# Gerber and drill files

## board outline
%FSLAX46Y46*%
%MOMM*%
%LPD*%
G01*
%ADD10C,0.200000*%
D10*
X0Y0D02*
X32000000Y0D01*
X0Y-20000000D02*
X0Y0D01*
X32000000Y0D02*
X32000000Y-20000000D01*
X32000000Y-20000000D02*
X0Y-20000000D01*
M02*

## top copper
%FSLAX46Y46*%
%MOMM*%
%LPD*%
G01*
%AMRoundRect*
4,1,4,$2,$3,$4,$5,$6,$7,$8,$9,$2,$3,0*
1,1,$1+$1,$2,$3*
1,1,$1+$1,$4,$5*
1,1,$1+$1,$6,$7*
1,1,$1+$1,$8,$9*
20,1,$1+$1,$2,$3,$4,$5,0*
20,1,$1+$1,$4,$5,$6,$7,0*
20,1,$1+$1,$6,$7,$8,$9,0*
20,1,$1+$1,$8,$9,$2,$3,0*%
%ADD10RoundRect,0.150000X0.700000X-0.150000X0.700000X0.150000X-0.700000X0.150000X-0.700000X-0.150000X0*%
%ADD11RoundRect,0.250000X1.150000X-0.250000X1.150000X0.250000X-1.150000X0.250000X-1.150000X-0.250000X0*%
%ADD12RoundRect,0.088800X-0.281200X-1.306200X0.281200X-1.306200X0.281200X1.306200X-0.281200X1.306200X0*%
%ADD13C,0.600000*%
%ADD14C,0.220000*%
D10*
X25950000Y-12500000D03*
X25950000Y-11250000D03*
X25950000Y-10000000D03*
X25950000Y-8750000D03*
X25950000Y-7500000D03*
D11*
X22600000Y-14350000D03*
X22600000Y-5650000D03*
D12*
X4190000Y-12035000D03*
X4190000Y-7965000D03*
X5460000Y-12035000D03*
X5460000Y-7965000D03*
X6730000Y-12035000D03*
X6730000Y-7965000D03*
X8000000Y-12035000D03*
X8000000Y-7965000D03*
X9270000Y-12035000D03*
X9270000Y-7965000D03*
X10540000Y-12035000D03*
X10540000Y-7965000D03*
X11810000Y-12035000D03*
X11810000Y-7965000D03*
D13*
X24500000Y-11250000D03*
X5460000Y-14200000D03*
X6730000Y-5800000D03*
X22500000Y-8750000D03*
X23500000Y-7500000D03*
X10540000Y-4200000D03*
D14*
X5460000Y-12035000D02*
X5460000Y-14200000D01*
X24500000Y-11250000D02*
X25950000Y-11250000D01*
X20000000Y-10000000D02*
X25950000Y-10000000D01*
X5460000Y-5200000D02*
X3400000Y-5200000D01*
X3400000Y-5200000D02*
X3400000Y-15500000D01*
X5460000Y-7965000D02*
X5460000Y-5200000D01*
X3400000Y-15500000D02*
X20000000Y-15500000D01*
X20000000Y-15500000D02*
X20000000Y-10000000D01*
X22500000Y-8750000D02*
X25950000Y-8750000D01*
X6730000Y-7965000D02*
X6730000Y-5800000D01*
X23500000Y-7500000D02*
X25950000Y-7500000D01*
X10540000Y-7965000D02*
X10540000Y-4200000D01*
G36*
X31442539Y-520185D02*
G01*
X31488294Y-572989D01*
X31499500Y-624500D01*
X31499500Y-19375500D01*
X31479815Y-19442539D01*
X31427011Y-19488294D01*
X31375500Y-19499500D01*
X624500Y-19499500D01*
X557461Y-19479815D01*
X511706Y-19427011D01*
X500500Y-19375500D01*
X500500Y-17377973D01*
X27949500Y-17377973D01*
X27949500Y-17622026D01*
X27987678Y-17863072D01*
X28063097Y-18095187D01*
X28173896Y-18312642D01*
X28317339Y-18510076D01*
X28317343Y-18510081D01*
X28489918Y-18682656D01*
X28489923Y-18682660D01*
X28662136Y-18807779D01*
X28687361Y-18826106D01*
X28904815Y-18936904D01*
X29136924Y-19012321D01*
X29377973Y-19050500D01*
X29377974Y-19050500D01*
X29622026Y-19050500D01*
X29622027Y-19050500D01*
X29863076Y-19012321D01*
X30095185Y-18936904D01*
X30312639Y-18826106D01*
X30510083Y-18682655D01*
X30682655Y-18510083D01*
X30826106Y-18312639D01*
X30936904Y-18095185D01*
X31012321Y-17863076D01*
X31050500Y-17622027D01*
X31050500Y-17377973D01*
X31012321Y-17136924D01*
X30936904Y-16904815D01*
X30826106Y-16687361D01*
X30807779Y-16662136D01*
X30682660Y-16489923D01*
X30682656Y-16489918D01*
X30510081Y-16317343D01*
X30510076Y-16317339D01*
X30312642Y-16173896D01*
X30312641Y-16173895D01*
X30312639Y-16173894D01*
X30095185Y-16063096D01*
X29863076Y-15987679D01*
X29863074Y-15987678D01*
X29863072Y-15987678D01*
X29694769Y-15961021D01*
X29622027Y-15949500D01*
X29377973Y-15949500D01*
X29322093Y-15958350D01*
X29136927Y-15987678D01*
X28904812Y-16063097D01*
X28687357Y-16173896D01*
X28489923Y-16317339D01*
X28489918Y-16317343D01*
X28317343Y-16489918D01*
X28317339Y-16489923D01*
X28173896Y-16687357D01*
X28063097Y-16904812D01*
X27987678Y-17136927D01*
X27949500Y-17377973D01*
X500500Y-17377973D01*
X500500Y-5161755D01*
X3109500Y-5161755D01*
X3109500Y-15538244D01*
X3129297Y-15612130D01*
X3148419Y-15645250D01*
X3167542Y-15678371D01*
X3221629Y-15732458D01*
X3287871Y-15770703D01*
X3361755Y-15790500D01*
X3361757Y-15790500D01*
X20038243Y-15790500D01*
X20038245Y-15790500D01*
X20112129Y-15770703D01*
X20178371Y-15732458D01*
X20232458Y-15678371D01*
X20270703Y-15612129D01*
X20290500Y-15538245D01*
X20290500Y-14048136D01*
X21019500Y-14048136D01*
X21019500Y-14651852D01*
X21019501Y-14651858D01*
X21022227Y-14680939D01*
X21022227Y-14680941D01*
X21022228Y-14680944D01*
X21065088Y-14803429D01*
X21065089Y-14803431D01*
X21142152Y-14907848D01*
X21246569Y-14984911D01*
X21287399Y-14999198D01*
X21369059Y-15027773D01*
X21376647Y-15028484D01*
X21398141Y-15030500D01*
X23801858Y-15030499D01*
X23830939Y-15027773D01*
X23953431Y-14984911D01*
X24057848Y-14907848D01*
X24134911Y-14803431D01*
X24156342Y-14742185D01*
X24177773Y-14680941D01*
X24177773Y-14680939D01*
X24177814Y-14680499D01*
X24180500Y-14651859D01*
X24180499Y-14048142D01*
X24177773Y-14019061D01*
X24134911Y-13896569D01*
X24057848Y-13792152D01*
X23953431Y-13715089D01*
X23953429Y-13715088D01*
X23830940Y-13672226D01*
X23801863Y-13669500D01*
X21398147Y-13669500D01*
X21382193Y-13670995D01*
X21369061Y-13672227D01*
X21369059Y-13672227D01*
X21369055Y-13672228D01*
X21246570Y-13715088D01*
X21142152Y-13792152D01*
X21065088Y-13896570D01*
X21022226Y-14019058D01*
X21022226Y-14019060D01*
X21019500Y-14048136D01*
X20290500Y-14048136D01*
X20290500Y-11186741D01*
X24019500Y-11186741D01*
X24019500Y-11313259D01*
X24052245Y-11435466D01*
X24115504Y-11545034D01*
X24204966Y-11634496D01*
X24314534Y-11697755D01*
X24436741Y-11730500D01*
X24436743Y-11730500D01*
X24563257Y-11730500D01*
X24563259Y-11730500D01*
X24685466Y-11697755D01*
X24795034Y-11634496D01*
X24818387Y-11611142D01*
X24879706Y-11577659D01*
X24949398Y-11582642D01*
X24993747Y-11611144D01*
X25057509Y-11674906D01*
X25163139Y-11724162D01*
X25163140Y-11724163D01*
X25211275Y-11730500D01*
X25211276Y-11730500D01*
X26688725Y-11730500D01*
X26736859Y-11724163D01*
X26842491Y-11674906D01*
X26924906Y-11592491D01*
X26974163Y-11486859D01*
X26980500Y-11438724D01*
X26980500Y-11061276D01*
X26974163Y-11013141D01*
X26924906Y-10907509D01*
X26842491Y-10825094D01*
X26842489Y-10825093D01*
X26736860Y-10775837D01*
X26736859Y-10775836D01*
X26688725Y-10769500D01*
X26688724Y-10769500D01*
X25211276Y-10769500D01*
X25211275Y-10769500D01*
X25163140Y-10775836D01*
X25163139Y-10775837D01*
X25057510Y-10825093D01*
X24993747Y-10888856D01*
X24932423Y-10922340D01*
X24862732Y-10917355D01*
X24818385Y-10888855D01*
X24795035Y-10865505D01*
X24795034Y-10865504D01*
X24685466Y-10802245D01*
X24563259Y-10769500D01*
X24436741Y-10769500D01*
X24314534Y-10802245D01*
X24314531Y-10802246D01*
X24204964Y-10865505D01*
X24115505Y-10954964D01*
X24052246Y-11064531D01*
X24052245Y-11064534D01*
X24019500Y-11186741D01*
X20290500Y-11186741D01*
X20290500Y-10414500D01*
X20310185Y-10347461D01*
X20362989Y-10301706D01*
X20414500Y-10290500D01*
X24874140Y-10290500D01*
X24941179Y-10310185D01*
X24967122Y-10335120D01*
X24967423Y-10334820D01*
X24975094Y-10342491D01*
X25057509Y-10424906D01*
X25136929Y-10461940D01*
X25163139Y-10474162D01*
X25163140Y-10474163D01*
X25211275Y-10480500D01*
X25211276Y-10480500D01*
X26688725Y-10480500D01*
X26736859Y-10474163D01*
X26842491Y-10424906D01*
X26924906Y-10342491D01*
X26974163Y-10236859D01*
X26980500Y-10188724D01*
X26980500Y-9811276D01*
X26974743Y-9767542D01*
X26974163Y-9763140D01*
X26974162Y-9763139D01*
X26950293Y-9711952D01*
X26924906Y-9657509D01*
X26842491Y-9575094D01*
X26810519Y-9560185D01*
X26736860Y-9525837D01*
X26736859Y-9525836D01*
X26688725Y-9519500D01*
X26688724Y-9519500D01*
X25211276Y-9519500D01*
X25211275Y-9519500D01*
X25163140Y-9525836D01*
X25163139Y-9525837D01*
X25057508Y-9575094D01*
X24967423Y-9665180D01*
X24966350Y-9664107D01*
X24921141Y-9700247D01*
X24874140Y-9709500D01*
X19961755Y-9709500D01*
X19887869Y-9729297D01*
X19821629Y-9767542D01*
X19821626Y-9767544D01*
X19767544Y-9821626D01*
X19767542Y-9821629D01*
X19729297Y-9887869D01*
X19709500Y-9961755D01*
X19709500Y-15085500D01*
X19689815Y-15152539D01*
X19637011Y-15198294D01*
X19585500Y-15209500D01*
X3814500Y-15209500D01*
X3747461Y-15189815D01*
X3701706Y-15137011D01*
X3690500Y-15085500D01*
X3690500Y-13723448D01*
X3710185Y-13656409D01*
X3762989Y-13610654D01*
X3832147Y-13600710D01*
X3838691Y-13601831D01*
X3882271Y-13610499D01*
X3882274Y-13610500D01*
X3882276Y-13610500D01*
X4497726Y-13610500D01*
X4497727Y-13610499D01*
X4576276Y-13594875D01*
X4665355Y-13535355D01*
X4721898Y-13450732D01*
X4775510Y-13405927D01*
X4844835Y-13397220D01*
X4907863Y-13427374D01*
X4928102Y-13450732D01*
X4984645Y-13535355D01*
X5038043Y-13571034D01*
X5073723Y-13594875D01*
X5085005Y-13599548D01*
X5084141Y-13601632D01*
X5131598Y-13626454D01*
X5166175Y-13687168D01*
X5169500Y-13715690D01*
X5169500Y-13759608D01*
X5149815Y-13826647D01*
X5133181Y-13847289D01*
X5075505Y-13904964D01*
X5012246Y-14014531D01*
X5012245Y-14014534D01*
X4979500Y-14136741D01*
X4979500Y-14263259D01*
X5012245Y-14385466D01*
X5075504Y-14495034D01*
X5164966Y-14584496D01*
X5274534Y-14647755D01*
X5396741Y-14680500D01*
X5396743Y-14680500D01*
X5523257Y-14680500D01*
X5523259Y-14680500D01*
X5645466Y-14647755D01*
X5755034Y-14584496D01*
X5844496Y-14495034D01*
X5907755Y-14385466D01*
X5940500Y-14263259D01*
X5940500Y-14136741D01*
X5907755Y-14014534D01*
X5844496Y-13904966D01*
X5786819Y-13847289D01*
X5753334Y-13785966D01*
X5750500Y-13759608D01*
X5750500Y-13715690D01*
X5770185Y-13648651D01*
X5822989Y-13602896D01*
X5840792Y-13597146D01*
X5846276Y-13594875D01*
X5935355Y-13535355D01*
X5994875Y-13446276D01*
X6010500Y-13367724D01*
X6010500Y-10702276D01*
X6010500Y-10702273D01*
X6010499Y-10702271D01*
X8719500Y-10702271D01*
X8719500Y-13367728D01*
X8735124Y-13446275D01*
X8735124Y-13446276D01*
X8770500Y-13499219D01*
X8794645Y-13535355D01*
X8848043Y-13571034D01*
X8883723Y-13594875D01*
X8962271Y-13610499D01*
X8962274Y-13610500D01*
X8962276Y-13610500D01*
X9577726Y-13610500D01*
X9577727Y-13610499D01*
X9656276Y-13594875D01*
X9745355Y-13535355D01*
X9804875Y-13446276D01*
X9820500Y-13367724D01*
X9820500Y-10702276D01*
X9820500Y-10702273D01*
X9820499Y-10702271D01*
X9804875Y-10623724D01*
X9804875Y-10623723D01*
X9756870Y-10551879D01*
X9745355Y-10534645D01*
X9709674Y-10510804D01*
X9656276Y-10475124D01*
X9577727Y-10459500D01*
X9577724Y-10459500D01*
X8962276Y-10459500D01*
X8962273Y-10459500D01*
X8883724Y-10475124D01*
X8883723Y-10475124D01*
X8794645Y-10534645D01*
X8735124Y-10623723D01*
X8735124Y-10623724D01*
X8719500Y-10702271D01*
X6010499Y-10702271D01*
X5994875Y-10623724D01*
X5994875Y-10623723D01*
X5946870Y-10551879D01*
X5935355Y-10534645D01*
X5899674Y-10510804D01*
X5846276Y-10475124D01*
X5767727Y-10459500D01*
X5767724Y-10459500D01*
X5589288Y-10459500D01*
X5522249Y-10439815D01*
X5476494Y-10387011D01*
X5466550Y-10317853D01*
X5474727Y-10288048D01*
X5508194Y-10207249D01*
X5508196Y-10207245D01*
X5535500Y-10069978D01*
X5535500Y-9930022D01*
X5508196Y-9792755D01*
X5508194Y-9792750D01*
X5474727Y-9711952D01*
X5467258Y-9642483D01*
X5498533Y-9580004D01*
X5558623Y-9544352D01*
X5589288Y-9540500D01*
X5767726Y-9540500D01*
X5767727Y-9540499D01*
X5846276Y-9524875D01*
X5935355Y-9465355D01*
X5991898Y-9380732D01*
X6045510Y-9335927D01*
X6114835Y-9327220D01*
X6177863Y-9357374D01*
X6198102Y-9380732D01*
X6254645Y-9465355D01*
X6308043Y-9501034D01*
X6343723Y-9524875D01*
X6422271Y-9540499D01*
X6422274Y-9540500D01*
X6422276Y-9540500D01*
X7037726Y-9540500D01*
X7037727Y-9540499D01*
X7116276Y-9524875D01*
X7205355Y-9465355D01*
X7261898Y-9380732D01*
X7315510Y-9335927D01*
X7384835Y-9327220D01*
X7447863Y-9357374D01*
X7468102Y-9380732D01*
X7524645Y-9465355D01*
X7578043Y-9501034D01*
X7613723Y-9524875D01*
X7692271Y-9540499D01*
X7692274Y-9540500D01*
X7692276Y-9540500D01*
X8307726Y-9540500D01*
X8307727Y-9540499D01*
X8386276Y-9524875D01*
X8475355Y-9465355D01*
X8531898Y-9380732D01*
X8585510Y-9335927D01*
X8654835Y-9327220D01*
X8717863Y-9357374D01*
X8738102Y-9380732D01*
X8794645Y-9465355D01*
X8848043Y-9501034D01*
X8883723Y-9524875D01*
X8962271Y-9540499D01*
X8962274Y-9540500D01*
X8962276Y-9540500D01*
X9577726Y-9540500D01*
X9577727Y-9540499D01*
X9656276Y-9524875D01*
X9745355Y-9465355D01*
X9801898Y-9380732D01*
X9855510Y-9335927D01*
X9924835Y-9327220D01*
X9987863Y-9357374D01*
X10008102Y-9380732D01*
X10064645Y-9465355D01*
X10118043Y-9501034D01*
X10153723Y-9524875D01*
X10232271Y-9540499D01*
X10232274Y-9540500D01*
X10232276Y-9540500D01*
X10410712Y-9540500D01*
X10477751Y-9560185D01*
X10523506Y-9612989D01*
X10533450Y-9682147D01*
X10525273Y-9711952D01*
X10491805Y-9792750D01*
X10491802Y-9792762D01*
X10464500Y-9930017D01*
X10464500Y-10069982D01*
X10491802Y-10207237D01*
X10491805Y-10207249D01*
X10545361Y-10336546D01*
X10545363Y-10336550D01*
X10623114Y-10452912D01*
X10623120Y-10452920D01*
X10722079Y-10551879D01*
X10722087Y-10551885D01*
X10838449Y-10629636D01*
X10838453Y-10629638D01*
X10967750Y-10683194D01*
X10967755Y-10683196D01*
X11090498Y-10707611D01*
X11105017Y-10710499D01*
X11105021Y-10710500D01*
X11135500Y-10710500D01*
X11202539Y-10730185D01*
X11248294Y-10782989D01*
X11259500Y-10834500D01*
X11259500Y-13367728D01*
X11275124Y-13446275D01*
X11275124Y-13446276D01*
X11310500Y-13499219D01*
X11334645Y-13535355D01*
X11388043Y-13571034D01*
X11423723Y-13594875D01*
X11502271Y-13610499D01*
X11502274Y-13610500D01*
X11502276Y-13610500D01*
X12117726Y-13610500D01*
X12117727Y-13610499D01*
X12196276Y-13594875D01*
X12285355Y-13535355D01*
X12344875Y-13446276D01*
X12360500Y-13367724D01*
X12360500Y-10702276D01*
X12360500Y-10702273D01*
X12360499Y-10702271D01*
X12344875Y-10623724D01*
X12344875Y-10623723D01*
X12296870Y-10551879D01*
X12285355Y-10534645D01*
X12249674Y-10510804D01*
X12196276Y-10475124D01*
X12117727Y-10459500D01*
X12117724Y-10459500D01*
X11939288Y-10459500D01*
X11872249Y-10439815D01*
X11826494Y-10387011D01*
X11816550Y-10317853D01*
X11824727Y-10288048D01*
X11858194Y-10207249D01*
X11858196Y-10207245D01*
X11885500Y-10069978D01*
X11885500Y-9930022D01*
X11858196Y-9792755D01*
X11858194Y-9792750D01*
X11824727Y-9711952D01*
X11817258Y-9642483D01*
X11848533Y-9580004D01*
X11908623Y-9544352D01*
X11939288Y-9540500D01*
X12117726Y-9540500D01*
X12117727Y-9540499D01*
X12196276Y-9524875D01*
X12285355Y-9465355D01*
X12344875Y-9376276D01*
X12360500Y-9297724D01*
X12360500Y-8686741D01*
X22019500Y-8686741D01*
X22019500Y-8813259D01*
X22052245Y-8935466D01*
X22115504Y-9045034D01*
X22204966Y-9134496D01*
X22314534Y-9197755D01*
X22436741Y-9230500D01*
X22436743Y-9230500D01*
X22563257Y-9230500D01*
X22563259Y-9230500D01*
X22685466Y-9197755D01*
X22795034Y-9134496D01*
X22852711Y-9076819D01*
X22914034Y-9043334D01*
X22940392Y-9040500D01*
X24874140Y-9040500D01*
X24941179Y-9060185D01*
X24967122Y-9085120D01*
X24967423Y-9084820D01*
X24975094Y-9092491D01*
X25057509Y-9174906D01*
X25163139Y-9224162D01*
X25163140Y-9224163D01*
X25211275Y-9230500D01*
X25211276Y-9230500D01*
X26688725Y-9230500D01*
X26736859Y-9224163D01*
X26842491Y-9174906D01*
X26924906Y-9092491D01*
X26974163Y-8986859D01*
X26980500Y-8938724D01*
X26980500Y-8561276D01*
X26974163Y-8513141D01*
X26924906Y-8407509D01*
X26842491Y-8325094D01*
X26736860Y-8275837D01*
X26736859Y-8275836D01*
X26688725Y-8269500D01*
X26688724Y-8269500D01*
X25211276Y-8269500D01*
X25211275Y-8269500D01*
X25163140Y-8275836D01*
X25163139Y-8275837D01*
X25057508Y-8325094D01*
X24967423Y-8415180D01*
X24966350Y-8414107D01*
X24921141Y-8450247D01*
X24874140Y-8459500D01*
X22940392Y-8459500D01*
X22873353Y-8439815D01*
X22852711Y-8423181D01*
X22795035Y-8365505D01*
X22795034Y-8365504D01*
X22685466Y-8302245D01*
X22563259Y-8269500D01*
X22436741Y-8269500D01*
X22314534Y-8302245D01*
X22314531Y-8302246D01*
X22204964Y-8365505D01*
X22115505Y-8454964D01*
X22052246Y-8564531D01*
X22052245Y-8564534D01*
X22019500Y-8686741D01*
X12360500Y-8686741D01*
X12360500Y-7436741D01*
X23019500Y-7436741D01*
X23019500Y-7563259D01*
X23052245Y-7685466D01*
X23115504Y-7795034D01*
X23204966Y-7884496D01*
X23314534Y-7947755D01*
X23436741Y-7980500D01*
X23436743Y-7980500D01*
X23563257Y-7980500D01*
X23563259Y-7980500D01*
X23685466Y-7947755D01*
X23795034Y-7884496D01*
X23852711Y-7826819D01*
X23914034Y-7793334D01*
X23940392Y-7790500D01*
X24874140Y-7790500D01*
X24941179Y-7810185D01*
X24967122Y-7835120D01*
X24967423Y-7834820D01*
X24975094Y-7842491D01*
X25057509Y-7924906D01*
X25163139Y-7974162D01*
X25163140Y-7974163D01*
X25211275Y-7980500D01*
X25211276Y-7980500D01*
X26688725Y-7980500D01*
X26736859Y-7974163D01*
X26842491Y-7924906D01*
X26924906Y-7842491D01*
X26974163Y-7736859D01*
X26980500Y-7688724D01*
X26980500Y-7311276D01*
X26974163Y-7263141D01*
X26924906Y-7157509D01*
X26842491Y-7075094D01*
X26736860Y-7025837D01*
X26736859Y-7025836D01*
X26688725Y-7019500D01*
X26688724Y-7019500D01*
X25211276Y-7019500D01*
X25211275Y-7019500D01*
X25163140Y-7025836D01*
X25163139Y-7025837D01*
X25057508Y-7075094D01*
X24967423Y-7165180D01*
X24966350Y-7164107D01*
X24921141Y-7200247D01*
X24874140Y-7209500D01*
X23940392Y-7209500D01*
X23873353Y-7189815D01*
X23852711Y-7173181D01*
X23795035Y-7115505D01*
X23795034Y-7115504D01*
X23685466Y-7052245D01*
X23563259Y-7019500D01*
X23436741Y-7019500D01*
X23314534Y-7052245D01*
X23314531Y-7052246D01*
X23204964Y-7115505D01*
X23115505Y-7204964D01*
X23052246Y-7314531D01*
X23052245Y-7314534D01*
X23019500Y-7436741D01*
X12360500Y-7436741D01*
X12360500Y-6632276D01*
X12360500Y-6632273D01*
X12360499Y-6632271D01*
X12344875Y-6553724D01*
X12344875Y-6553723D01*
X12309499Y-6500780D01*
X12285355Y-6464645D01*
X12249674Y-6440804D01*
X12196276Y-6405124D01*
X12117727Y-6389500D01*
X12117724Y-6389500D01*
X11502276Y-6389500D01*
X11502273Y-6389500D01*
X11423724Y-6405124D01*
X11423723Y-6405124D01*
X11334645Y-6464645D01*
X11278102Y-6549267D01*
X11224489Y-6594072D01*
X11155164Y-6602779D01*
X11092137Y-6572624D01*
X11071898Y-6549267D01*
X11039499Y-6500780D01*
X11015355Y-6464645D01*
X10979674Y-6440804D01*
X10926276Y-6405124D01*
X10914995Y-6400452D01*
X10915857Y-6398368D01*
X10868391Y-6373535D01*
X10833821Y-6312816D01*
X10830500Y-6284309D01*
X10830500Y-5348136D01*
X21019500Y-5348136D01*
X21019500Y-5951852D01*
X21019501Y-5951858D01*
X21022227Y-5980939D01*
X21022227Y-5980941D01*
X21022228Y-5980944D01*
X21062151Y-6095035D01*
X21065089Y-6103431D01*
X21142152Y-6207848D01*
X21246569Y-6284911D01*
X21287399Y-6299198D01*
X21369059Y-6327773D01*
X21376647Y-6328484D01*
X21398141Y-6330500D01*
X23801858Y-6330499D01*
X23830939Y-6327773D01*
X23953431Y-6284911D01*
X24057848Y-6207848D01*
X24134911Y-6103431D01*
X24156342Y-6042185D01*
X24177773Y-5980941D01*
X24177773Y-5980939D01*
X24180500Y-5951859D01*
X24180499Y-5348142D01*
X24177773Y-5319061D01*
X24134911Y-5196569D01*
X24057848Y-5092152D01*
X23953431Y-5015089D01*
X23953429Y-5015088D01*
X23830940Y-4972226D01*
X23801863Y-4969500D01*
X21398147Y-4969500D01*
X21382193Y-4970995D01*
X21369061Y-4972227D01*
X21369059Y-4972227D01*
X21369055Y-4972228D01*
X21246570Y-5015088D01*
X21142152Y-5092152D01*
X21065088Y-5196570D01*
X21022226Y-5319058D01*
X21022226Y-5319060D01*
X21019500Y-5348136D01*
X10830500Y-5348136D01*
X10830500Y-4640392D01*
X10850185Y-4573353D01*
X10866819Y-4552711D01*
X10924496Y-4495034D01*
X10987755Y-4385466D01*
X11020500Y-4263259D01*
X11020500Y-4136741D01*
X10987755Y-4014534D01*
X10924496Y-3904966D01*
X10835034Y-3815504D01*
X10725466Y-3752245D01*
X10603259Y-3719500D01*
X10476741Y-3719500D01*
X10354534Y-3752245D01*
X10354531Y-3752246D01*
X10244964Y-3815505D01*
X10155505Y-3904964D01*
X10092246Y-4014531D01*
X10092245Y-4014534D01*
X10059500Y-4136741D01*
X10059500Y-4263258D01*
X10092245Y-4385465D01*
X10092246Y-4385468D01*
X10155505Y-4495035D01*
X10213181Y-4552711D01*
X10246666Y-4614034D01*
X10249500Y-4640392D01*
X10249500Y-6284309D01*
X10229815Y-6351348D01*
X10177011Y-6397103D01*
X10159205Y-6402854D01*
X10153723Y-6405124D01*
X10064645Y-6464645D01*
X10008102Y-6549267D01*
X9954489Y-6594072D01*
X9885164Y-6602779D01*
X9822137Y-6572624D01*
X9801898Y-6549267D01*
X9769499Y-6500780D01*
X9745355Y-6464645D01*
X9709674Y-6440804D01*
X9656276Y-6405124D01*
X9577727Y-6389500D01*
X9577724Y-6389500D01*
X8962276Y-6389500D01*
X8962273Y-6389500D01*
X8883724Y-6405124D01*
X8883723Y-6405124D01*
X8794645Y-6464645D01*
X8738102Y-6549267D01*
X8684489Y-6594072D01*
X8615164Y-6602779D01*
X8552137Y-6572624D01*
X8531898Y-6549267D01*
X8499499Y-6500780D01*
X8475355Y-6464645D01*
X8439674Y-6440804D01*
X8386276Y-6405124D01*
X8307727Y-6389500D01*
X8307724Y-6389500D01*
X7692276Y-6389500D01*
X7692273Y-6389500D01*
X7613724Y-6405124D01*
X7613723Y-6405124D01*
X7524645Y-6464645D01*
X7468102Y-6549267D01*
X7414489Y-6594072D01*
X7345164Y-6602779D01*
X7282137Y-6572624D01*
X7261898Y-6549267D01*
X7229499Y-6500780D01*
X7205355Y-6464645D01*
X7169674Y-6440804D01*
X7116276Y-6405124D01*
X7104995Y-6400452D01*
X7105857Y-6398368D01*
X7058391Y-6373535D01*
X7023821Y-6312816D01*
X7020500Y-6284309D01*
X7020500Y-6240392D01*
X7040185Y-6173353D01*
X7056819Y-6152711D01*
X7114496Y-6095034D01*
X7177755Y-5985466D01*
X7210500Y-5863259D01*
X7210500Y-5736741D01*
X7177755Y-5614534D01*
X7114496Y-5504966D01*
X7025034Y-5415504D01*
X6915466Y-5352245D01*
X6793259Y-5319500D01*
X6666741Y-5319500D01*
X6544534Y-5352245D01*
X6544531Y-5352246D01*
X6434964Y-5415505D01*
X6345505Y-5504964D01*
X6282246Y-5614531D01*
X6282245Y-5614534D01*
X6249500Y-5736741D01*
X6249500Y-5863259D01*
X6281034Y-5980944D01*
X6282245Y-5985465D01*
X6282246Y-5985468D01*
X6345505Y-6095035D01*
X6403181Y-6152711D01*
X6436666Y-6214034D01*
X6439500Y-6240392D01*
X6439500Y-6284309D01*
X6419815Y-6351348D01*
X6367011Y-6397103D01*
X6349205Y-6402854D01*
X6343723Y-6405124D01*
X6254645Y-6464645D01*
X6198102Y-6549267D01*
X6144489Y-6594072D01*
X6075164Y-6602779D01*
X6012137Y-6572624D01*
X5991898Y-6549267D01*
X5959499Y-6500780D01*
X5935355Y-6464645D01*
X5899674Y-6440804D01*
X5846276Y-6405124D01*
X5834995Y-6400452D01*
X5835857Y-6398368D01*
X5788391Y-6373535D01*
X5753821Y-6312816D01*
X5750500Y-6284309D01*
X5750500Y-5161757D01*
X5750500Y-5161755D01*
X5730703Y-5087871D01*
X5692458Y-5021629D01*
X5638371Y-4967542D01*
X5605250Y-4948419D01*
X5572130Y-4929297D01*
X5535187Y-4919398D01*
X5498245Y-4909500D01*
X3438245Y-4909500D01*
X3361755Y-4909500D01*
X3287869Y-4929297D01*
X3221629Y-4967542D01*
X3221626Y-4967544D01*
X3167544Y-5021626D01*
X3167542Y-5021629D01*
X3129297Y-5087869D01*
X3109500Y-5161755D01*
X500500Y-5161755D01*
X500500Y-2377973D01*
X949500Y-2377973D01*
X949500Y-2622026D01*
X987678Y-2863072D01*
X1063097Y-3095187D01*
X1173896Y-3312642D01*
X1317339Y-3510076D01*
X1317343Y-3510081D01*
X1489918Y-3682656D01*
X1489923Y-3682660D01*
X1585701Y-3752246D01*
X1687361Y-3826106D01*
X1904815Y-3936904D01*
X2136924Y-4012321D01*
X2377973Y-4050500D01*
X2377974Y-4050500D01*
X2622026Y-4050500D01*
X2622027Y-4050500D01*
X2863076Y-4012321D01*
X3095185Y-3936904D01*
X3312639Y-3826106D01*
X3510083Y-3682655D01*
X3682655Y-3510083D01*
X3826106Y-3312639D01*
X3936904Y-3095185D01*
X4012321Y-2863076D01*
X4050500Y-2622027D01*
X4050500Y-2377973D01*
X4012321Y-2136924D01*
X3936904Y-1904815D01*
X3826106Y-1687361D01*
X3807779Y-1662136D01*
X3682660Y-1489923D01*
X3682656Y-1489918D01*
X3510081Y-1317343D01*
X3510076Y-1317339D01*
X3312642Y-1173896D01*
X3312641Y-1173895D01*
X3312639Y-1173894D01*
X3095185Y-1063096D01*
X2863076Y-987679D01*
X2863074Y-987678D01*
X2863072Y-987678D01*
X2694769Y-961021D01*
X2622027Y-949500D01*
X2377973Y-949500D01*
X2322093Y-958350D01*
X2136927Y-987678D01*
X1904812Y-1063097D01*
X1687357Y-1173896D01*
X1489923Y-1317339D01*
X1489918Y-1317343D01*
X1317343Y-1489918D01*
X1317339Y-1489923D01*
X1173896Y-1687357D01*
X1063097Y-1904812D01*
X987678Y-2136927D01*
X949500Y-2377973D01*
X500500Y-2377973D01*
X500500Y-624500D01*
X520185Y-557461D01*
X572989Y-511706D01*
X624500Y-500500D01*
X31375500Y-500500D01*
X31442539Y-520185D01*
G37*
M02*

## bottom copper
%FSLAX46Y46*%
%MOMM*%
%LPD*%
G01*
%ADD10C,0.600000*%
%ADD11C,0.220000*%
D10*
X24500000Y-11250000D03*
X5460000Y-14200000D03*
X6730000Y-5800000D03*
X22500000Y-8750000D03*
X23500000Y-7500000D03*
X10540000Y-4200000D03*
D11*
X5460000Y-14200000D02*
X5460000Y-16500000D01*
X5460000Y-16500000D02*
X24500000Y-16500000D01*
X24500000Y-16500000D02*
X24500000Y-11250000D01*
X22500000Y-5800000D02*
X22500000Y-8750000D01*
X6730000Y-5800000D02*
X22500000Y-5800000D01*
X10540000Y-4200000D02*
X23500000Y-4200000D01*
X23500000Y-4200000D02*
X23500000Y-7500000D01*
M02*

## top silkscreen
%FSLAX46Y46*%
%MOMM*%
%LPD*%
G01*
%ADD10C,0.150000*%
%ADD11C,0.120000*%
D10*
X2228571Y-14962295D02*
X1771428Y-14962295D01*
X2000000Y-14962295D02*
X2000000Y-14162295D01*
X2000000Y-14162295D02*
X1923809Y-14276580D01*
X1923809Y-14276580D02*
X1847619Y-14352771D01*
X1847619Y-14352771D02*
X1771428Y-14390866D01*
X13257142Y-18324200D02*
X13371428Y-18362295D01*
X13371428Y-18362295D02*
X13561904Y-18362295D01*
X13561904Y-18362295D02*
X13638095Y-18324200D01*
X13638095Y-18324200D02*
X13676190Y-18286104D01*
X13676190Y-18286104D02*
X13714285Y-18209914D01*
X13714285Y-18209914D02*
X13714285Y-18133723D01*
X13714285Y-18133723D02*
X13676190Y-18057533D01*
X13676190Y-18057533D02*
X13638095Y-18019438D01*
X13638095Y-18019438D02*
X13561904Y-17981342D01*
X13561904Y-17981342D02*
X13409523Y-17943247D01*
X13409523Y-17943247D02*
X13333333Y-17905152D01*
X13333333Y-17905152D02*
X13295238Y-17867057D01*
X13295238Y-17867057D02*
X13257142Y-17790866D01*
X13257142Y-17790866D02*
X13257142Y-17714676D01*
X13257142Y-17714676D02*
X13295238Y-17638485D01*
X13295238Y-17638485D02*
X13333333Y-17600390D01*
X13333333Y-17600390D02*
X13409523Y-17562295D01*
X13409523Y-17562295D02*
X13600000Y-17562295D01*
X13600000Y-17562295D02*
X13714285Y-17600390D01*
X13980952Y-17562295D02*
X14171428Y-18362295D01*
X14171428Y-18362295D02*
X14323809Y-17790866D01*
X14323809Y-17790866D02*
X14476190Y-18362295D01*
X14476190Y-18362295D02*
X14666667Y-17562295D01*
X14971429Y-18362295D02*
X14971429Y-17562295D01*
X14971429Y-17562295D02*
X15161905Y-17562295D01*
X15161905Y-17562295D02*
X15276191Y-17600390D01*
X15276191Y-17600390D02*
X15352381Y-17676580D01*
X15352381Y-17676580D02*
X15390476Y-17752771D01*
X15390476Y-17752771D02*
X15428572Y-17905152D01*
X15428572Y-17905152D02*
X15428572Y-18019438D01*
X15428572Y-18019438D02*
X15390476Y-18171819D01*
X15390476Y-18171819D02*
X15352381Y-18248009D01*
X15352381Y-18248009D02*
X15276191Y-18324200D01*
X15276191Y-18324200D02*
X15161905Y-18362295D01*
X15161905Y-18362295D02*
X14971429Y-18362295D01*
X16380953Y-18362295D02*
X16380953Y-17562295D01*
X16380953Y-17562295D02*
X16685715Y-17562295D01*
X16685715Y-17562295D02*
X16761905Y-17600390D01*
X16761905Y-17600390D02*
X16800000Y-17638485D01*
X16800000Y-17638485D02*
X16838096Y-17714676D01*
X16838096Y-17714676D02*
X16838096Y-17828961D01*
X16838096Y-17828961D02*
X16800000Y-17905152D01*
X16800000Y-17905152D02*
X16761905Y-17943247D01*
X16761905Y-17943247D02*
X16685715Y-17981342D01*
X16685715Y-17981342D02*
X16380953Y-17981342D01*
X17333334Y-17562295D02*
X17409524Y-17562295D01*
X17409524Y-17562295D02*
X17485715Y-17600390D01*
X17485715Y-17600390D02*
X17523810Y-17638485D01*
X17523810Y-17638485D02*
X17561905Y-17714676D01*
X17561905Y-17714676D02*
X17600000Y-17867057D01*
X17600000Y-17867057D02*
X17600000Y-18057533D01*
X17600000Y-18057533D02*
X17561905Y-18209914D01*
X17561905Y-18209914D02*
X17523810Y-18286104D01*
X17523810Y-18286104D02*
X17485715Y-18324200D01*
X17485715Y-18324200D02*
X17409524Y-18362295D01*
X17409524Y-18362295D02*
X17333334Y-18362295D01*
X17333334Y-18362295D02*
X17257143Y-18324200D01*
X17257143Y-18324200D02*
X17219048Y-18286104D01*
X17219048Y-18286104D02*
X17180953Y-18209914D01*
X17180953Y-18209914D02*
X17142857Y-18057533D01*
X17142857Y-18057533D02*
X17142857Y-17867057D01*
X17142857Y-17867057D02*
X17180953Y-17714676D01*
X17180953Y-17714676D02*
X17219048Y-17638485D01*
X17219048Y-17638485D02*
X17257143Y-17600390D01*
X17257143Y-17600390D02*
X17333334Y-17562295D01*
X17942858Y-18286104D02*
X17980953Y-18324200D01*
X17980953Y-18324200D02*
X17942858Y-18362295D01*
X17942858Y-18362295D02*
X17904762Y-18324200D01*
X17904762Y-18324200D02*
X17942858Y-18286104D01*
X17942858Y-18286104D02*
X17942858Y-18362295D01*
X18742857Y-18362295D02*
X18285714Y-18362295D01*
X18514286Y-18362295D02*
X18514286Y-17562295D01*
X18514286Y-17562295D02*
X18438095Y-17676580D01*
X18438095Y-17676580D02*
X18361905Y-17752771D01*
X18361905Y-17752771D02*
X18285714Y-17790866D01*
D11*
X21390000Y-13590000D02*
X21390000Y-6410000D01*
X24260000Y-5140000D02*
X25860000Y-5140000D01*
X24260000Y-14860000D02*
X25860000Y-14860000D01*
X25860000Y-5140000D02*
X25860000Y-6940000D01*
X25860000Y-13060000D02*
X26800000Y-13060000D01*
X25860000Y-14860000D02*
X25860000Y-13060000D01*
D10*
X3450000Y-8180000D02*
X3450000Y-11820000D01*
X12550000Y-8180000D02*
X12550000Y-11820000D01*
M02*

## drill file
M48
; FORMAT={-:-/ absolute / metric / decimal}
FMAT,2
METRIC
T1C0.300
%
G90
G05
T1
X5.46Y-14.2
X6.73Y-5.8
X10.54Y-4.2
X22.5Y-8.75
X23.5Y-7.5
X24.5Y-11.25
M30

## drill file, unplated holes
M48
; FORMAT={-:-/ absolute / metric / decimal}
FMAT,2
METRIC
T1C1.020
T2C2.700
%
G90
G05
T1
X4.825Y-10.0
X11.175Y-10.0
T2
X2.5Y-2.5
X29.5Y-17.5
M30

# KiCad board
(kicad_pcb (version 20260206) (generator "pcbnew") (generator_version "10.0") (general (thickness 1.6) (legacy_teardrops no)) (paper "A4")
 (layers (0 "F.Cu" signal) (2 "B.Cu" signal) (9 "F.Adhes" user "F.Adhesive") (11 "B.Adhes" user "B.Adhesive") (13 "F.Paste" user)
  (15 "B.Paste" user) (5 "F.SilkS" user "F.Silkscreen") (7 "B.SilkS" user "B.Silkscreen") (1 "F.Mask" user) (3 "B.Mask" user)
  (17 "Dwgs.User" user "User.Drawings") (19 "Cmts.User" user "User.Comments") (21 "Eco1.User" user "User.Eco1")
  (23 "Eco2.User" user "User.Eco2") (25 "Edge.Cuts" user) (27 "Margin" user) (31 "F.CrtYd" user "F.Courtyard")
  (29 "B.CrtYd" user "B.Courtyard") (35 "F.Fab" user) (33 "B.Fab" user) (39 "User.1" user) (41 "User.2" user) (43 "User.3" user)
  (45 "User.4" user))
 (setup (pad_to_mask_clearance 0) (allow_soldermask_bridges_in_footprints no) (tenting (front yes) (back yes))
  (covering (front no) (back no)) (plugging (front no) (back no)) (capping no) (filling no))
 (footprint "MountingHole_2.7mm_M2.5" (layer "F.Cu") (at 2.5 2.5)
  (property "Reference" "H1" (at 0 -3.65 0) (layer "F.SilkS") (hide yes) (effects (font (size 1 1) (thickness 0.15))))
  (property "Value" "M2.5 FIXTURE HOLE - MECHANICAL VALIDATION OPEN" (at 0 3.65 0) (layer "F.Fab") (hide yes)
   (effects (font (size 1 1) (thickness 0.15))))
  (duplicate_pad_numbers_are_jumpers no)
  (pad "" np_thru_hole circle (at 0 0) (size 2.7 2.7) (drill 2.7) (layers "*.Cu" "*.Mask")))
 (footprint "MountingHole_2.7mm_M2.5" (layer "F.Cu") (at 29.5 17.5)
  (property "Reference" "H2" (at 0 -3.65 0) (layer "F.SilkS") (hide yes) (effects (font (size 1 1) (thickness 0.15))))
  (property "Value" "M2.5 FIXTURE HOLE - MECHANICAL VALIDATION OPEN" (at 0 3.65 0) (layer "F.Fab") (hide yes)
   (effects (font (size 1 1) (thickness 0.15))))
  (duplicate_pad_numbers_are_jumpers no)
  (pad "" np_thru_hole circle (at 0 0) (size 2.7 2.7) (drill 2.7) (layers "*.Cu" "*.Mask")))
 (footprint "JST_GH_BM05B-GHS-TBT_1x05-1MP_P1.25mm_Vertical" (layer "F.Cu") (at 24 10 90)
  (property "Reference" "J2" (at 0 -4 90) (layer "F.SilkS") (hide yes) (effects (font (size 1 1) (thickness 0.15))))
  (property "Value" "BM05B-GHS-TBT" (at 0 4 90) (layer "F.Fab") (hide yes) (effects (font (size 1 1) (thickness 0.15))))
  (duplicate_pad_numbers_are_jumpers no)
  (fp_line (start -3.59 -2.61) (end 3.59 -2.61) (stroke (width 0.12) (type solid)) (layer "F.SilkS"))
  (fp_line (start 4.86 0.26) (end 4.86 1.86) (stroke (width 0.12) (type solid)) (layer "F.SilkS"))
  (fp_line (start -4.86 0.26) (end -4.86 1.86) (stroke (width 0.12) (type solid)) (layer "F.SilkS"))
  (fp_line (start 4.86 1.86) (end 3.06 1.86) (stroke (width 0.12) (type solid)) (layer "F.SilkS"))
  (fp_line (start -3.06 1.86) (end -3.06 2.8) (stroke (width 0.12) (type solid)) (layer "F.SilkS"))
  (fp_line (start -4.86 1.86) (end -3.06 1.86) (stroke (width 0.12) (type solid)) (layer "F.SilkS"))
  (pad "1" smd roundrect (at -2.5 1.95 90) (size 0.6 1.7) (layers "F.Cu" "F.Mask" "F.Paste") (roundrect_rratio 0.25) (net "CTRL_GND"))
  (pad "2" smd roundrect (at -1.25 1.95 90) (size 0.6 1.7) (layers "F.Cu" "F.Mask" "F.Paste") (roundrect_rratio 0.25) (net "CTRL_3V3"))
  (pad "3" smd roundrect (at 0 1.95 90) (size 0.6 1.7) (layers "F.Cu" "F.Mask" "F.Paste") (roundrect_rratio 0.25) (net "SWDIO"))
  (pad "4" smd roundrect (at 1.25 1.95 90) (size 0.6 1.7) (layers "F.Cu" "F.Mask" "F.Paste") (roundrect_rratio 0.25) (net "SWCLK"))
  (pad "5" smd roundrect (at 2.5 1.95 90) (size 0.6 1.7) (layers "F.Cu" "F.Mask" "F.Paste") (roundrect_rratio 0.25) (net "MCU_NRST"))
  (pad "MP" smd roundrect (at -4.35 -1.4 90) (size 1 2.8) (layers "F.Cu" "F.Mask" "F.Paste") (roundrect_rratio 0.25))
  (pad "MP" smd roundrect (at 4.35 -1.4 90) (size 1 2.8) (layers "F.Cu" "F.Mask" "F.Paste") (roundrect_rratio 0.25)))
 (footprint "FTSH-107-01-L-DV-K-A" (layer "F.Cu") (at 8 10)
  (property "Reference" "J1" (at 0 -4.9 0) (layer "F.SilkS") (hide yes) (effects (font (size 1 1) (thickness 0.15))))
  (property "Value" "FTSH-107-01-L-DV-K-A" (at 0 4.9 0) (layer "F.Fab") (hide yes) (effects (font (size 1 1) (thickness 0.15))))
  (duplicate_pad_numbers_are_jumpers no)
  (fp_line (start -4.55 -1.82) (end -4.55 1.82) (stroke (width 0.15) (type solid)) (layer "F.SilkS"))
  (fp_line (start 4.55 -1.82) (end 4.55 1.82) (stroke (width 0.15) (type solid)) (layer "F.SilkS"))
  (pad "" np_thru_hole circle (at -3.175 0) (size 1.02 1.02) (drill 1.02) (layers "*.Cu" "*.Mask"))
  (pad "" np_thru_hole circle (at 3.175 0) (size 1.02 1.02) (drill 1.02) (layers "*.Cu" "*.Mask"))
  (pad "1" smd roundrect (at -3.81 2.035) (size 0.74 2.79) (layers "F.Cu" "F.Mask" "F.Paste") (roundrect_rratio 0.12))
  (pad "2" smd roundrect (at -3.81 -2.035) (size 0.74 2.79) (layers "F.Cu" "F.Mask" "F.Paste") (roundrect_rratio 0.12))
  (pad "3" smd roundrect (at -2.54 2.035) (size 0.74 2.79) (layers "F.Cu" "F.Mask" "F.Paste") (roundrect_rratio 0.12) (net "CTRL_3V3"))
  (pad "4" smd roundrect (at -2.54 -2.035) (size 0.74 2.79) (layers "F.Cu" "F.Mask" "F.Paste") (roundrect_rratio 0.12) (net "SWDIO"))
  (pad "5" smd roundrect (at -1.27 2.035) (size 0.74 2.79) (layers "F.Cu" "F.Mask" "F.Paste") (roundrect_rratio 0.12) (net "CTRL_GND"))
  (pad "6" smd roundrect (at -1.27 -2.035) (size 0.74 2.79) (layers "F.Cu" "F.Mask" "F.Paste") (roundrect_rratio 0.12) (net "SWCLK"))
  (pad "7" smd roundrect (at 0 2.035) (size 0.74 2.79) (layers "F.Cu" "F.Mask" "F.Paste") (roundrect_rratio 0.12) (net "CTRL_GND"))
  (pad "8" smd roundrect (at 0 -2.035) (size 0.74 2.79) (layers "F.Cu" "F.Mask" "F.Paste") (roundrect_rratio 0.12))
  (pad "9" smd roundrect (at 1.27 2.035) (size 0.74 2.79) (layers "F.Cu" "F.Mask" "F.Paste") (roundrect_rratio 0.12))
  (pad "10" smd roundrect (at 1.27 -2.035) (size 0.74 2.79) (layers "F.Cu" "F.Mask" "F.Paste") (roundrect_rratio 0.12))
  (pad "11" smd roundrect (at 2.54 2.035) (size 0.74 2.79) (layers "F.Cu" "F.Mask" "F.Paste") (roundrect_rratio 0.12) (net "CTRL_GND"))
  (pad "12" smd roundrect (at 2.54 -2.035) (size 0.74 2.79) (layers "F.Cu" "F.Mask" "F.Paste") (roundrect_rratio 0.12) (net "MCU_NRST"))
  (pad "13" smd roundrect (at 3.81 2.035) (size 0.74 2.79) (layers "F.Cu" "F.Mask" "F.Paste") (roundrect_rratio 0.12))
  (pad "14" smd roundrect (at 3.81 -2.035) (size 0.74 2.79) (layers "F.Cu" "F.Mask" "F.Paste") (roundrect_rratio 0.12)))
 (gr_line (start 0 0) (end 32 0) (stroke (width 0.2) (type default)) (layer "Edge.Cuts"))
 (gr_line (start 0 20) (end 0 0) (stroke (width 0.2) (type default)) (layer "Edge.Cuts"))
 (gr_line (start 32 0) (end 32 20) (stroke (width 0.2) (type default)) (layer "Edge.Cuts"))
 (gr_line (start 32 20) (end 0 20) (stroke (width 0.2) (type default)) (layer "Edge.Cuts"))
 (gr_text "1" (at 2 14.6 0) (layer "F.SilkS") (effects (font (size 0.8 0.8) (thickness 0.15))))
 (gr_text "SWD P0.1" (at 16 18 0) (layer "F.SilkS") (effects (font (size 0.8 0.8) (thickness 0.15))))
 (segment (start 5.46 12.035) (end 5.46 14.2) (width 0.22) (layer "F.Cu") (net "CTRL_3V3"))
 (segment (start 24.5 11.25) (end 25.95 11.25) (width 0.22) (layer "F.Cu") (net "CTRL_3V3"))
 (via (at 24.5 11.25) (size 0.6) (drill 0.3) (layers "F.Cu" "B.Cu") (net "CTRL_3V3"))
 (via (at 5.46 14.2) (size 0.6) (drill 0.3) (layers "F.Cu" "B.Cu") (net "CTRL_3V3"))
 (segment (start 5.46 14.2) (end 5.46 16.5) (width 0.22) (layer "B.Cu") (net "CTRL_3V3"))
 (segment (start 5.46 16.5) (end 24.5 16.5) (width 0.22) (layer "B.Cu") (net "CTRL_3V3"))
 (segment (start 24.5 16.5) (end 24.5 11.25) (width 0.22) (layer "B.Cu") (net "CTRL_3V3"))
 (segment (start 20 10) (end 25.95 10) (width 0.22) (layer "F.Cu") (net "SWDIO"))
 (segment (start 5.46 5.2) (end 3.4 5.2) (width 0.22) (layer "F.Cu") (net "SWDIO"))
 (segment (start 3.4 5.2) (end 3.4 15.5) (width 0.22) (layer "F.Cu") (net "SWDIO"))
 (segment (start 5.46 7.965) (end 5.46 5.2) (width 0.22) (layer "F.Cu") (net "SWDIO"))
 (segment (start 3.4 15.5) (end 20 15.5) (width 0.22) (layer "F.Cu") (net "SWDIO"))
 (segment (start 20 15.5) (end 20 10) (width 0.22) (layer "F.Cu") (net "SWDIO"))
 (segment (start 22.5 8.75) (end 25.95 8.75) (width 0.22) (layer "F.Cu") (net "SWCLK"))
 (segment (start 6.73 7.965) (end 6.73 5.8) (width 0.22) (layer "F.Cu") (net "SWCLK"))
 (via (at 6.73 5.8) (size 0.6) (drill 0.3) (layers "F.Cu" "B.Cu") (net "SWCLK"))
 (via (at 22.5 8.75) (size 0.6) (drill 0.3) (layers "F.Cu" "B.Cu") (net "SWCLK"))
 (segment (start 22.5 5.8) (end 22.5 8.75) (width 0.22) (layer "B.Cu") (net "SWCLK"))
 (segment (start 6.73 5.8) (end 22.5 5.8) (width 0.22) (layer "B.Cu") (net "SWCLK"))
 (segment (start 23.5 7.5) (end 25.95 7.5) (width 0.22) (layer "F.Cu") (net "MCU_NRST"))
 (segment (start 10.54 7.965) (end 10.54 4.2) (width 0.22) (layer "F.Cu") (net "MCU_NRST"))
 (via (at 23.5 7.5) (size 0.6) (drill 0.3) (layers "F.Cu" "B.Cu") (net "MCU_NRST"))
 (via (at 10.54 4.2) (size 0.6) (drill 0.3) (layers "F.Cu" "B.Cu") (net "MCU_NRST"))
 (segment (start 10.54 4.2) (end 23.5 4.2) (width 0.22) (layer "B.Cu") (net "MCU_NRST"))
 (segment (start 23.5 4.2) (end 23.5 7.5) (width 0.22) (layer "B.Cu") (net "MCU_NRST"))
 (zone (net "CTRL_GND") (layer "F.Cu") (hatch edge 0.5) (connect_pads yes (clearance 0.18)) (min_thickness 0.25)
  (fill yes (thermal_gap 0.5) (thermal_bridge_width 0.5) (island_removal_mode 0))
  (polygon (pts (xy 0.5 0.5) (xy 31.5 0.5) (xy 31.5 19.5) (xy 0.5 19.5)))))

